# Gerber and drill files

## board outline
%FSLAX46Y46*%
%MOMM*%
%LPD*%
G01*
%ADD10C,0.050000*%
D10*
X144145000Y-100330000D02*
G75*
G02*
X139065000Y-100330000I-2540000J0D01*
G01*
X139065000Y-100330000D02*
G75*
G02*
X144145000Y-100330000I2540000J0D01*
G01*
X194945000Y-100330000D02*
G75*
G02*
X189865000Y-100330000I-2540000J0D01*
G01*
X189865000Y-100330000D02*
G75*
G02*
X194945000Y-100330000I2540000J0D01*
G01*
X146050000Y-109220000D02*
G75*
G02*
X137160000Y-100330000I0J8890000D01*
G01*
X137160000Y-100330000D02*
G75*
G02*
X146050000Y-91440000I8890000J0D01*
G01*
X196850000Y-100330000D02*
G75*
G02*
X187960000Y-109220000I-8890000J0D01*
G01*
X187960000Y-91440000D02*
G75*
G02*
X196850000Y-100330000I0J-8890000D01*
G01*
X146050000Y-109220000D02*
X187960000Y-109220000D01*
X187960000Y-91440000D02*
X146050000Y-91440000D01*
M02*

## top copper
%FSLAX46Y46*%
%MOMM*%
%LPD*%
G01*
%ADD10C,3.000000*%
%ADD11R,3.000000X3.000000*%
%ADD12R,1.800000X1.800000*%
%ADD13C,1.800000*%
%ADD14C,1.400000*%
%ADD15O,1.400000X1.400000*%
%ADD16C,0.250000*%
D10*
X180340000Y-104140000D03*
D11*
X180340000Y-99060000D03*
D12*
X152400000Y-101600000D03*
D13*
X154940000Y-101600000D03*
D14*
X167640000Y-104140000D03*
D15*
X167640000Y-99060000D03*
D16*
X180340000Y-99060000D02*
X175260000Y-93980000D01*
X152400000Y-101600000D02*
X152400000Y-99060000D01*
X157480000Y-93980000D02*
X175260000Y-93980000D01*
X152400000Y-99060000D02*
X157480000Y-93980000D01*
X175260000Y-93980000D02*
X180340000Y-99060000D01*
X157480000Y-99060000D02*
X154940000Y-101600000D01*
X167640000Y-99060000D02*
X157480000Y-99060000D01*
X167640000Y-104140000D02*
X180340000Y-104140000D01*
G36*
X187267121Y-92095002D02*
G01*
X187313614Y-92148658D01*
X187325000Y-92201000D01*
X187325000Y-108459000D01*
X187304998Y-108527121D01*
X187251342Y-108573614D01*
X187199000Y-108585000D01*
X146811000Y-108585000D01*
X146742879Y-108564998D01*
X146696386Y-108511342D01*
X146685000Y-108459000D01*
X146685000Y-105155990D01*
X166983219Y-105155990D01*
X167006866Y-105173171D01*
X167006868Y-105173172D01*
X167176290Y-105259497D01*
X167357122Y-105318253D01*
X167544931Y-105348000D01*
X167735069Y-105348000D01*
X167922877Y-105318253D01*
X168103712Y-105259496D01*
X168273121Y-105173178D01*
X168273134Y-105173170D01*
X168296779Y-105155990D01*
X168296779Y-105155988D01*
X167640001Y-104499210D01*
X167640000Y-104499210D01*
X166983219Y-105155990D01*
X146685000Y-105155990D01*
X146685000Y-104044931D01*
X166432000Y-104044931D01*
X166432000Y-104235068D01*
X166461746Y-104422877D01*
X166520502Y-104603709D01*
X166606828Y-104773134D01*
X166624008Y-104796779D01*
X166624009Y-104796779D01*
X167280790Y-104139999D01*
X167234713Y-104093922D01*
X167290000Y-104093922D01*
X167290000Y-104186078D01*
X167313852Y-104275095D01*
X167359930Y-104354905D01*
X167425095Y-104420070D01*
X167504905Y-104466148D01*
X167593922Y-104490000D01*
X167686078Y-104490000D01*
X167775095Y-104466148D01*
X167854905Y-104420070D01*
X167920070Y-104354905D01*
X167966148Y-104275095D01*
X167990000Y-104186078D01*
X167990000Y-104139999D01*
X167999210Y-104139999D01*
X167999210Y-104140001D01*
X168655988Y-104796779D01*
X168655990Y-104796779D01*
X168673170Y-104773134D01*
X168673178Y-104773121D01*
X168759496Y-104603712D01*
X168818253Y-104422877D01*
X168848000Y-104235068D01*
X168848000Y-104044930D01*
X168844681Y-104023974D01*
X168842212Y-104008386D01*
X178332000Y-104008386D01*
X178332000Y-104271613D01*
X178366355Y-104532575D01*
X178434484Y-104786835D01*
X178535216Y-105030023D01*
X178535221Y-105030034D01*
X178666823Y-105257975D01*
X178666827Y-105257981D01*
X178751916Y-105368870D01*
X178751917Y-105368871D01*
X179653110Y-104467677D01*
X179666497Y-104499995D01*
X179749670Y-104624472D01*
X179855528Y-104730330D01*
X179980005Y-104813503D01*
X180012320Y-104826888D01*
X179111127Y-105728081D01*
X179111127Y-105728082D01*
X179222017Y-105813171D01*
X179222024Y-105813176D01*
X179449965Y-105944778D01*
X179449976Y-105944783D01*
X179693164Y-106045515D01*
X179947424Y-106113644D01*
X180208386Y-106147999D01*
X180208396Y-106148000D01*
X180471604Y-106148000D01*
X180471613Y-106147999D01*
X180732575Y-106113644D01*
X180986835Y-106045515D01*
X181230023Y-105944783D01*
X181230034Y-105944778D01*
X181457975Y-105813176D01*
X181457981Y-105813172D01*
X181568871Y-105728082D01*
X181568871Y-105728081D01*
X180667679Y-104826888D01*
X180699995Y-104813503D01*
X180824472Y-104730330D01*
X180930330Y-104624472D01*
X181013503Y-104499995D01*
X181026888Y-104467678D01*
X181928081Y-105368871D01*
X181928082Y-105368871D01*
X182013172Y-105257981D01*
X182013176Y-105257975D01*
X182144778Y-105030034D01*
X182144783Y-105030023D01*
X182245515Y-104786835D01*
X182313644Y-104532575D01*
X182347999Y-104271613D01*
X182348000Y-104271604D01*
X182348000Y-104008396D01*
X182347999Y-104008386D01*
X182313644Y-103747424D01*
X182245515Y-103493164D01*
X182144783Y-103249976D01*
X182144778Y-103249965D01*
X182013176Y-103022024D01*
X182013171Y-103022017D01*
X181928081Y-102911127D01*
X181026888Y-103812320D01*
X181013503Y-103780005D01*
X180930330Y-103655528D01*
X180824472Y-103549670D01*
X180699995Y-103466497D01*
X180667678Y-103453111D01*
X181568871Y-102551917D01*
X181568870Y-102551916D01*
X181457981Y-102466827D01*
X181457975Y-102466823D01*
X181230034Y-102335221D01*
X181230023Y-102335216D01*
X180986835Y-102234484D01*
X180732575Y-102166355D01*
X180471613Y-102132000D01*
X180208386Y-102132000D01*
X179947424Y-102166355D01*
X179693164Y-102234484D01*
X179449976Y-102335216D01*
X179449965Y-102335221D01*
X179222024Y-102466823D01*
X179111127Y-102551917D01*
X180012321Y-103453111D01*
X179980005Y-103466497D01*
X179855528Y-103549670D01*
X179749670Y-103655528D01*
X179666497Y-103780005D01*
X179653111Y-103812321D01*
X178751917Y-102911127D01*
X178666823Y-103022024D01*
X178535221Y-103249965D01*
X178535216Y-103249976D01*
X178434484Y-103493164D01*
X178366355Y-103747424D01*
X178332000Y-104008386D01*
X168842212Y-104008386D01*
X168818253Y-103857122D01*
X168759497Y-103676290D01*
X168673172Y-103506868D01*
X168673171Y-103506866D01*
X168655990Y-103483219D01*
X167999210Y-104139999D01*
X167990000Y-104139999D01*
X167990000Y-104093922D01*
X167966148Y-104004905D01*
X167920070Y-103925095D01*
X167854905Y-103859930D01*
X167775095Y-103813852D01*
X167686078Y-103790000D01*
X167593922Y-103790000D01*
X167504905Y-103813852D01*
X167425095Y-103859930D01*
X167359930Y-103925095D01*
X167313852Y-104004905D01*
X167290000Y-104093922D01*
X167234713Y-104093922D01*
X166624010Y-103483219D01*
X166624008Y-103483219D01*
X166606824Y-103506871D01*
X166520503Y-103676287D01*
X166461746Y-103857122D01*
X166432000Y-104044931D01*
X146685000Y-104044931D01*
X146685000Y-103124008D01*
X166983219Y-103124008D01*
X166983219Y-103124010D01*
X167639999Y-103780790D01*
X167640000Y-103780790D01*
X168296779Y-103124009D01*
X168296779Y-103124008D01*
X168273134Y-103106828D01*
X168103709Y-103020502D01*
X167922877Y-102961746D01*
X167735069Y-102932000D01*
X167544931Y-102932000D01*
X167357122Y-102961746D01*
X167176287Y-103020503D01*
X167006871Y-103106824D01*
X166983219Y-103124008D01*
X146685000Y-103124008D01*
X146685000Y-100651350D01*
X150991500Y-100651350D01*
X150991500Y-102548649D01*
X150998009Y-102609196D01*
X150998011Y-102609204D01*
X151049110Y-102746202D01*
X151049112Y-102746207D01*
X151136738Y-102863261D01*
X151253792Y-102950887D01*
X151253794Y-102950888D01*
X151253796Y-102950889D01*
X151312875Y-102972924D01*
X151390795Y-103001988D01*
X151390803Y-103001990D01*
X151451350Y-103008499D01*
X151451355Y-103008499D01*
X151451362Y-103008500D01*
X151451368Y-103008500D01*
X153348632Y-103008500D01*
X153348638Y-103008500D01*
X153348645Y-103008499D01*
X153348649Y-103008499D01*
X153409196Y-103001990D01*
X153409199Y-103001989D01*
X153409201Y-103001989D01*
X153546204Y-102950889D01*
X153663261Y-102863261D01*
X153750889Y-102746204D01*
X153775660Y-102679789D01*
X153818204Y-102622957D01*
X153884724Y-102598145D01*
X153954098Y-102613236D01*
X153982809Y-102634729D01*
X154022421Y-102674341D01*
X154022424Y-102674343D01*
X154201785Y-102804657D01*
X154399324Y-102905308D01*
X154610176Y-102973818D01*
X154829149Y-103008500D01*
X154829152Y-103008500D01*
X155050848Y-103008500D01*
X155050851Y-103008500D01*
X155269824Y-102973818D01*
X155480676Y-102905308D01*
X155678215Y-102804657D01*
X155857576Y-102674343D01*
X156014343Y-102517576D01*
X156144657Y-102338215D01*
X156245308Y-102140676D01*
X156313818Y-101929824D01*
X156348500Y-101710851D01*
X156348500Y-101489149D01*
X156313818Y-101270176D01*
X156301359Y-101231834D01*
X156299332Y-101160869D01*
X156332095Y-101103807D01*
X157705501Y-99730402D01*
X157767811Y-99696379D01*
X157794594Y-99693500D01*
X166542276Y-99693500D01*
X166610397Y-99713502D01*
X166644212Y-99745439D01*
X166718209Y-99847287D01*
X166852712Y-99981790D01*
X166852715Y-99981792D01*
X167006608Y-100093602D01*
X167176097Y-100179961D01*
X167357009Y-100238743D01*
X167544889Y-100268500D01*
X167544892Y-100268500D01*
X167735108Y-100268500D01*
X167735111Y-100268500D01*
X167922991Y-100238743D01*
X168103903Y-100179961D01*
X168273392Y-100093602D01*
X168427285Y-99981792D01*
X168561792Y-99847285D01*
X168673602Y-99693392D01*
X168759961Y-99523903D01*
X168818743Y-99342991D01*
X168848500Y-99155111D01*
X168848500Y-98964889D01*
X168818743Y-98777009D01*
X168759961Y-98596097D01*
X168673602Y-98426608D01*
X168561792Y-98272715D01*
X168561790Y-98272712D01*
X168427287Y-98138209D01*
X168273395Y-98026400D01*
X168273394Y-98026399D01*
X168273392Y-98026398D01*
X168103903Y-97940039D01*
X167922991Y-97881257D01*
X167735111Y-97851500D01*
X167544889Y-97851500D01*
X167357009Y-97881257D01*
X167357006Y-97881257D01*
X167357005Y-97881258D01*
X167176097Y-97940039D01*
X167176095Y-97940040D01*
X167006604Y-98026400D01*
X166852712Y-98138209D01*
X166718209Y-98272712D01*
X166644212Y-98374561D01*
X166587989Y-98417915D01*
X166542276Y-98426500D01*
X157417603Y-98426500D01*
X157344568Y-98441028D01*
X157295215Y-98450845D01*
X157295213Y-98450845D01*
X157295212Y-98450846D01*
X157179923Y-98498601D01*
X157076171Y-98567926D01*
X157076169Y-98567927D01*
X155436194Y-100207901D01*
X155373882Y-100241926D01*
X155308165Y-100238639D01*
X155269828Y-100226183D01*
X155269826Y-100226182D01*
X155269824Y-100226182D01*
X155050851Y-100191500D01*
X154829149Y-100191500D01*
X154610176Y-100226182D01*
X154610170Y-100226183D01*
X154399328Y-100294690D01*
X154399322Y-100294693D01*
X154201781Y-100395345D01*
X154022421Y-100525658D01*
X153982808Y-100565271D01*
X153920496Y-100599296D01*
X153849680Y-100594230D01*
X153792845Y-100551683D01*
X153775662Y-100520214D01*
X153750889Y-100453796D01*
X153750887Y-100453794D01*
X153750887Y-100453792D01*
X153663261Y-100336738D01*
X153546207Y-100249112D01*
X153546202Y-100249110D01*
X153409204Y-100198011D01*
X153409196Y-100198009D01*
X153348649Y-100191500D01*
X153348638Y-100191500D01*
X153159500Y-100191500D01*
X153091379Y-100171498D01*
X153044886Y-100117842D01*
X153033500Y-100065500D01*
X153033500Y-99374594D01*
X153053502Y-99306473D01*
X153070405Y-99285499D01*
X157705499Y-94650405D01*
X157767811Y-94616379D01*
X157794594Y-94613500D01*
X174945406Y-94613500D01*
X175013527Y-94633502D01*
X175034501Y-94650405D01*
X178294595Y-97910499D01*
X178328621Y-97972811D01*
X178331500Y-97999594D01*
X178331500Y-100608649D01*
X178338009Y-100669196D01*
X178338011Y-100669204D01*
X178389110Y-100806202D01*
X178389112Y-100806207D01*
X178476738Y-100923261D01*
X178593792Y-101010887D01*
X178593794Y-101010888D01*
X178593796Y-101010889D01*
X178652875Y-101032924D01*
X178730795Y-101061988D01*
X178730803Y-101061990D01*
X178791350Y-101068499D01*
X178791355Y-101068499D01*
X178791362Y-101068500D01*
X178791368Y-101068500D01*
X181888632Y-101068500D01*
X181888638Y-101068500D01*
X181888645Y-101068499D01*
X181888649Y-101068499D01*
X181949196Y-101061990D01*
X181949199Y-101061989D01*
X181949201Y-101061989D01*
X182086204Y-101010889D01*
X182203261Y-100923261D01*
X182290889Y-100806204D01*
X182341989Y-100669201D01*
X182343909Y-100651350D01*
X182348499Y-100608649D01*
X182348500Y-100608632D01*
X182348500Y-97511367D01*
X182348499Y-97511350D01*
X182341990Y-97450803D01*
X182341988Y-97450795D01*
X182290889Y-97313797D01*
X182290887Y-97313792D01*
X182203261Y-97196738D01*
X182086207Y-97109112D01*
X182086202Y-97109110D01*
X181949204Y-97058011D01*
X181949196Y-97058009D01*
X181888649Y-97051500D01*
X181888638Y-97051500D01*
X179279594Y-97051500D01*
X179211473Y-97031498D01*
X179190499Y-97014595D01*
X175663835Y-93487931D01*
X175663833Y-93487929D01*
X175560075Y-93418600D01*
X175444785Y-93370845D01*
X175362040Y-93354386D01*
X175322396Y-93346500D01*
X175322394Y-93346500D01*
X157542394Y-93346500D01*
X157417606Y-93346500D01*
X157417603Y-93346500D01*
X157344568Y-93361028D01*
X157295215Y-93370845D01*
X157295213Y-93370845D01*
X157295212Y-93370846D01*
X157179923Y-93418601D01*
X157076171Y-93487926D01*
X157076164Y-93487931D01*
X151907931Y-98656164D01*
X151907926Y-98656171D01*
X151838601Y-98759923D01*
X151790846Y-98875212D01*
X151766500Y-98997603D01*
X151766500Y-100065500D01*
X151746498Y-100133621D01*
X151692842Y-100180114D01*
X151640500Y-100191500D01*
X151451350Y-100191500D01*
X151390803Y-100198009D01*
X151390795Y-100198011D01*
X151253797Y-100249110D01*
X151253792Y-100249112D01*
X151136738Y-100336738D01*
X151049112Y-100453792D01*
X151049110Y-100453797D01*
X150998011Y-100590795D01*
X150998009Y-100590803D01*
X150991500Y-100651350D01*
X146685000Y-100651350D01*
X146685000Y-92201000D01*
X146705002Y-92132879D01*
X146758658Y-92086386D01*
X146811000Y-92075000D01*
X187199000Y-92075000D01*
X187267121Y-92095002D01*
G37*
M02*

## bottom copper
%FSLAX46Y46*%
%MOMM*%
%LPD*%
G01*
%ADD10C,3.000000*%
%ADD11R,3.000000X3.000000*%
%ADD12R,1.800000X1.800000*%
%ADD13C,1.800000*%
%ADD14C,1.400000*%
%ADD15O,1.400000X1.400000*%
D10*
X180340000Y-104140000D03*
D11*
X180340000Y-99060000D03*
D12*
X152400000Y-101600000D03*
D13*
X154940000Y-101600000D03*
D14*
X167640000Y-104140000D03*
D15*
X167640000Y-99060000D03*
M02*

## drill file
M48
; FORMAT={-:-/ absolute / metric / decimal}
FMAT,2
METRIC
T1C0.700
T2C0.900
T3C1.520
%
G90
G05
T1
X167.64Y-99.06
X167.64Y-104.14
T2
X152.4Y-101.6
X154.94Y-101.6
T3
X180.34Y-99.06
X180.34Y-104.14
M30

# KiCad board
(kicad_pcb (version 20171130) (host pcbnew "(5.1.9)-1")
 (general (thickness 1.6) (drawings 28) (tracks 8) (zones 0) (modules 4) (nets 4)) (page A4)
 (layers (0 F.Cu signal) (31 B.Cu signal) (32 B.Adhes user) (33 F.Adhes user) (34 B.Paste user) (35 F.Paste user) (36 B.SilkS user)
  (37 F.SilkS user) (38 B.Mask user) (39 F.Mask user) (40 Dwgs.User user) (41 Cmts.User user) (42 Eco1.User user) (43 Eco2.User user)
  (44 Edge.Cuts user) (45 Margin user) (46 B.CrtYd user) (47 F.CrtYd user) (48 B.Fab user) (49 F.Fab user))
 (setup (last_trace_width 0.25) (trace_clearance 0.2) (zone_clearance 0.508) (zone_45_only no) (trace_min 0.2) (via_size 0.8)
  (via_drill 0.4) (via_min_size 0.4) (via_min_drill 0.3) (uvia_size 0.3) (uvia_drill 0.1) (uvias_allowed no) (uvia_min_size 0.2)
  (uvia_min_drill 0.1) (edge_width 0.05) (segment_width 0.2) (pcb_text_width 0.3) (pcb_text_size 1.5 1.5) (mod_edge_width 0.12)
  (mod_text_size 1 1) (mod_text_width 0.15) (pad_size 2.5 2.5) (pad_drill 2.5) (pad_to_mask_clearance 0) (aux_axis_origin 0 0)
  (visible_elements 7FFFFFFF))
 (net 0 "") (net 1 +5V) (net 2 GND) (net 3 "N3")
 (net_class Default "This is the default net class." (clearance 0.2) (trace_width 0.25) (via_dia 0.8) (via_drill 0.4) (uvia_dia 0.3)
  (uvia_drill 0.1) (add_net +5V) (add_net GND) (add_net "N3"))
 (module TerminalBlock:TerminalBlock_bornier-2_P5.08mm (layer F.Cu) (at 180.34 99.06 270)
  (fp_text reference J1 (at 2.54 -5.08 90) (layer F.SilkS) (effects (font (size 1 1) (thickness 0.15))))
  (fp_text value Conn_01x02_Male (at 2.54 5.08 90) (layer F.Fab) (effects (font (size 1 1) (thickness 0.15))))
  (pad 2 thru_hole circle (at 5.08 0 270) (size 3 3) (drill 1.52) (layers *.Cu *.Mask) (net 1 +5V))
  (pad 1 thru_hole rect (at 0 0 270) (size 3 3) (drill 1.52) (layers *.Cu *.Mask) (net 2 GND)))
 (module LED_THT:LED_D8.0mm (layer F.Cu) (at 152.4 101.6)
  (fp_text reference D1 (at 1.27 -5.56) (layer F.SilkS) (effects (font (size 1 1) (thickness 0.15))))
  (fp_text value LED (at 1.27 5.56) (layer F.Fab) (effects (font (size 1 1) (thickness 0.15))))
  (pad 1 thru_hole rect (at 0 0) (size 1.8 1.8) (drill 0.9) (layers *.Cu *.Mask) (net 2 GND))
  (pad 2 thru_hole circle (at 2.54 0) (size 1.8 1.8) (drill 0.9) (layers *.Cu *.Mask) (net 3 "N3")))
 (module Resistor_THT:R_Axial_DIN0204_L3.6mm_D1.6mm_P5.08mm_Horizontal (layer F.Cu) (at 167.64 104.14 90)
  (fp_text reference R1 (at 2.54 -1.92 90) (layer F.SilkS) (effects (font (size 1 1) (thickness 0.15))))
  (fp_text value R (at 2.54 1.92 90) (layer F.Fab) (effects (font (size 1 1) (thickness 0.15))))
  (pad 1 thru_hole circle (at 0 0 90) (size 1.4 1.4) (drill 0.7) (layers *.Cu *.Mask) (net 1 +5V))
  (pad 2 thru_hole oval (at 5.08 0 90) (size 1.4 1.4) (drill 0.7) (layers *.Cu *.Mask) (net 3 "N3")))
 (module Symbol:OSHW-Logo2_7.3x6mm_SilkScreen (layer B.Cu) (at 161.29 99.695 180)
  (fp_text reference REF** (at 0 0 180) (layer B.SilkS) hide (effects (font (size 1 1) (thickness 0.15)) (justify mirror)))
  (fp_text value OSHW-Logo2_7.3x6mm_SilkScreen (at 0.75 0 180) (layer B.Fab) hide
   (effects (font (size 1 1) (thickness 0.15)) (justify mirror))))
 (gr_circle (center 141.605 100.33) (end 139.065 100.33) (layer Edge.Cuts) (width 0.05))
 (gr_circle (center 192.405 100.33) (end 194.945 100.33) (layer Edge.Cuts) (width 0.05))
 (gr_arc (start 146.05 100.33) (end 146.05 109.22) (angle 90) (layer Edge.Cuts) (width 0.05))
 (gr_arc (start 146.05 100.33) (end 137.16 100.33) (angle 90) (layer Edge.Cuts) (width 0.05))
 (gr_arc (start 187.96 100.33) (end 196.85 100.33) (angle 90) (layer Edge.Cuts) (width 0.05))
 (gr_arc (start 187.96 100.33) (end 187.96 91.44) (angle 90) (layer Edge.Cuts) (width 0.05))
 (gr_line (start 146.05 109.22) (end 187.96 109.22) (angle 90) (layer Edge.Cuts) (width 0.05))
 (gr_line (start 187.96 91.44) (end 146.05 91.44) (angle 90) (layer Edge.Cuts) (width 0.05))
 (segment (start 180.34 99.06) (end 175.26 93.98) (width 0.25) (layer F.Cu) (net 2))
 (segment (start 152.4 101.6) (end 152.4 99.06) (width 0.25) (layer F.Cu) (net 2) (status 400000))
 (segment (start 157.48 93.98) (end 175.26 93.98) (width 0.25) (layer F.Cu) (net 2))
 (segment (start 152.4 99.06) (end 157.48 93.98) (width 0.25) (layer F.Cu) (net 2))
 (segment (start 175.26 93.98) (end 180.34 99.06) (width 0.25) (layer F.Cu) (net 2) (status 800000))
 (segment (start 157.48 99.06) (end 154.94 101.6) (width 0.25) (layer F.Cu) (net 3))
 (segment (start 167.64 99.06) (end 157.48 99.06) (width 0.25) (layer F.Cu) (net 3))
 (segment (start 167.64 104.14) (end 180.34 104.14) (width 0.25) (layer F.Cu) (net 1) (status C00000))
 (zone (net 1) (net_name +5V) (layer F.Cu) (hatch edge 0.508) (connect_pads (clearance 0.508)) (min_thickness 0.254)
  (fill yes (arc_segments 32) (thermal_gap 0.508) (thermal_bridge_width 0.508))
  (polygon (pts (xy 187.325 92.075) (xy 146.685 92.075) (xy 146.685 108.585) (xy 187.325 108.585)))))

